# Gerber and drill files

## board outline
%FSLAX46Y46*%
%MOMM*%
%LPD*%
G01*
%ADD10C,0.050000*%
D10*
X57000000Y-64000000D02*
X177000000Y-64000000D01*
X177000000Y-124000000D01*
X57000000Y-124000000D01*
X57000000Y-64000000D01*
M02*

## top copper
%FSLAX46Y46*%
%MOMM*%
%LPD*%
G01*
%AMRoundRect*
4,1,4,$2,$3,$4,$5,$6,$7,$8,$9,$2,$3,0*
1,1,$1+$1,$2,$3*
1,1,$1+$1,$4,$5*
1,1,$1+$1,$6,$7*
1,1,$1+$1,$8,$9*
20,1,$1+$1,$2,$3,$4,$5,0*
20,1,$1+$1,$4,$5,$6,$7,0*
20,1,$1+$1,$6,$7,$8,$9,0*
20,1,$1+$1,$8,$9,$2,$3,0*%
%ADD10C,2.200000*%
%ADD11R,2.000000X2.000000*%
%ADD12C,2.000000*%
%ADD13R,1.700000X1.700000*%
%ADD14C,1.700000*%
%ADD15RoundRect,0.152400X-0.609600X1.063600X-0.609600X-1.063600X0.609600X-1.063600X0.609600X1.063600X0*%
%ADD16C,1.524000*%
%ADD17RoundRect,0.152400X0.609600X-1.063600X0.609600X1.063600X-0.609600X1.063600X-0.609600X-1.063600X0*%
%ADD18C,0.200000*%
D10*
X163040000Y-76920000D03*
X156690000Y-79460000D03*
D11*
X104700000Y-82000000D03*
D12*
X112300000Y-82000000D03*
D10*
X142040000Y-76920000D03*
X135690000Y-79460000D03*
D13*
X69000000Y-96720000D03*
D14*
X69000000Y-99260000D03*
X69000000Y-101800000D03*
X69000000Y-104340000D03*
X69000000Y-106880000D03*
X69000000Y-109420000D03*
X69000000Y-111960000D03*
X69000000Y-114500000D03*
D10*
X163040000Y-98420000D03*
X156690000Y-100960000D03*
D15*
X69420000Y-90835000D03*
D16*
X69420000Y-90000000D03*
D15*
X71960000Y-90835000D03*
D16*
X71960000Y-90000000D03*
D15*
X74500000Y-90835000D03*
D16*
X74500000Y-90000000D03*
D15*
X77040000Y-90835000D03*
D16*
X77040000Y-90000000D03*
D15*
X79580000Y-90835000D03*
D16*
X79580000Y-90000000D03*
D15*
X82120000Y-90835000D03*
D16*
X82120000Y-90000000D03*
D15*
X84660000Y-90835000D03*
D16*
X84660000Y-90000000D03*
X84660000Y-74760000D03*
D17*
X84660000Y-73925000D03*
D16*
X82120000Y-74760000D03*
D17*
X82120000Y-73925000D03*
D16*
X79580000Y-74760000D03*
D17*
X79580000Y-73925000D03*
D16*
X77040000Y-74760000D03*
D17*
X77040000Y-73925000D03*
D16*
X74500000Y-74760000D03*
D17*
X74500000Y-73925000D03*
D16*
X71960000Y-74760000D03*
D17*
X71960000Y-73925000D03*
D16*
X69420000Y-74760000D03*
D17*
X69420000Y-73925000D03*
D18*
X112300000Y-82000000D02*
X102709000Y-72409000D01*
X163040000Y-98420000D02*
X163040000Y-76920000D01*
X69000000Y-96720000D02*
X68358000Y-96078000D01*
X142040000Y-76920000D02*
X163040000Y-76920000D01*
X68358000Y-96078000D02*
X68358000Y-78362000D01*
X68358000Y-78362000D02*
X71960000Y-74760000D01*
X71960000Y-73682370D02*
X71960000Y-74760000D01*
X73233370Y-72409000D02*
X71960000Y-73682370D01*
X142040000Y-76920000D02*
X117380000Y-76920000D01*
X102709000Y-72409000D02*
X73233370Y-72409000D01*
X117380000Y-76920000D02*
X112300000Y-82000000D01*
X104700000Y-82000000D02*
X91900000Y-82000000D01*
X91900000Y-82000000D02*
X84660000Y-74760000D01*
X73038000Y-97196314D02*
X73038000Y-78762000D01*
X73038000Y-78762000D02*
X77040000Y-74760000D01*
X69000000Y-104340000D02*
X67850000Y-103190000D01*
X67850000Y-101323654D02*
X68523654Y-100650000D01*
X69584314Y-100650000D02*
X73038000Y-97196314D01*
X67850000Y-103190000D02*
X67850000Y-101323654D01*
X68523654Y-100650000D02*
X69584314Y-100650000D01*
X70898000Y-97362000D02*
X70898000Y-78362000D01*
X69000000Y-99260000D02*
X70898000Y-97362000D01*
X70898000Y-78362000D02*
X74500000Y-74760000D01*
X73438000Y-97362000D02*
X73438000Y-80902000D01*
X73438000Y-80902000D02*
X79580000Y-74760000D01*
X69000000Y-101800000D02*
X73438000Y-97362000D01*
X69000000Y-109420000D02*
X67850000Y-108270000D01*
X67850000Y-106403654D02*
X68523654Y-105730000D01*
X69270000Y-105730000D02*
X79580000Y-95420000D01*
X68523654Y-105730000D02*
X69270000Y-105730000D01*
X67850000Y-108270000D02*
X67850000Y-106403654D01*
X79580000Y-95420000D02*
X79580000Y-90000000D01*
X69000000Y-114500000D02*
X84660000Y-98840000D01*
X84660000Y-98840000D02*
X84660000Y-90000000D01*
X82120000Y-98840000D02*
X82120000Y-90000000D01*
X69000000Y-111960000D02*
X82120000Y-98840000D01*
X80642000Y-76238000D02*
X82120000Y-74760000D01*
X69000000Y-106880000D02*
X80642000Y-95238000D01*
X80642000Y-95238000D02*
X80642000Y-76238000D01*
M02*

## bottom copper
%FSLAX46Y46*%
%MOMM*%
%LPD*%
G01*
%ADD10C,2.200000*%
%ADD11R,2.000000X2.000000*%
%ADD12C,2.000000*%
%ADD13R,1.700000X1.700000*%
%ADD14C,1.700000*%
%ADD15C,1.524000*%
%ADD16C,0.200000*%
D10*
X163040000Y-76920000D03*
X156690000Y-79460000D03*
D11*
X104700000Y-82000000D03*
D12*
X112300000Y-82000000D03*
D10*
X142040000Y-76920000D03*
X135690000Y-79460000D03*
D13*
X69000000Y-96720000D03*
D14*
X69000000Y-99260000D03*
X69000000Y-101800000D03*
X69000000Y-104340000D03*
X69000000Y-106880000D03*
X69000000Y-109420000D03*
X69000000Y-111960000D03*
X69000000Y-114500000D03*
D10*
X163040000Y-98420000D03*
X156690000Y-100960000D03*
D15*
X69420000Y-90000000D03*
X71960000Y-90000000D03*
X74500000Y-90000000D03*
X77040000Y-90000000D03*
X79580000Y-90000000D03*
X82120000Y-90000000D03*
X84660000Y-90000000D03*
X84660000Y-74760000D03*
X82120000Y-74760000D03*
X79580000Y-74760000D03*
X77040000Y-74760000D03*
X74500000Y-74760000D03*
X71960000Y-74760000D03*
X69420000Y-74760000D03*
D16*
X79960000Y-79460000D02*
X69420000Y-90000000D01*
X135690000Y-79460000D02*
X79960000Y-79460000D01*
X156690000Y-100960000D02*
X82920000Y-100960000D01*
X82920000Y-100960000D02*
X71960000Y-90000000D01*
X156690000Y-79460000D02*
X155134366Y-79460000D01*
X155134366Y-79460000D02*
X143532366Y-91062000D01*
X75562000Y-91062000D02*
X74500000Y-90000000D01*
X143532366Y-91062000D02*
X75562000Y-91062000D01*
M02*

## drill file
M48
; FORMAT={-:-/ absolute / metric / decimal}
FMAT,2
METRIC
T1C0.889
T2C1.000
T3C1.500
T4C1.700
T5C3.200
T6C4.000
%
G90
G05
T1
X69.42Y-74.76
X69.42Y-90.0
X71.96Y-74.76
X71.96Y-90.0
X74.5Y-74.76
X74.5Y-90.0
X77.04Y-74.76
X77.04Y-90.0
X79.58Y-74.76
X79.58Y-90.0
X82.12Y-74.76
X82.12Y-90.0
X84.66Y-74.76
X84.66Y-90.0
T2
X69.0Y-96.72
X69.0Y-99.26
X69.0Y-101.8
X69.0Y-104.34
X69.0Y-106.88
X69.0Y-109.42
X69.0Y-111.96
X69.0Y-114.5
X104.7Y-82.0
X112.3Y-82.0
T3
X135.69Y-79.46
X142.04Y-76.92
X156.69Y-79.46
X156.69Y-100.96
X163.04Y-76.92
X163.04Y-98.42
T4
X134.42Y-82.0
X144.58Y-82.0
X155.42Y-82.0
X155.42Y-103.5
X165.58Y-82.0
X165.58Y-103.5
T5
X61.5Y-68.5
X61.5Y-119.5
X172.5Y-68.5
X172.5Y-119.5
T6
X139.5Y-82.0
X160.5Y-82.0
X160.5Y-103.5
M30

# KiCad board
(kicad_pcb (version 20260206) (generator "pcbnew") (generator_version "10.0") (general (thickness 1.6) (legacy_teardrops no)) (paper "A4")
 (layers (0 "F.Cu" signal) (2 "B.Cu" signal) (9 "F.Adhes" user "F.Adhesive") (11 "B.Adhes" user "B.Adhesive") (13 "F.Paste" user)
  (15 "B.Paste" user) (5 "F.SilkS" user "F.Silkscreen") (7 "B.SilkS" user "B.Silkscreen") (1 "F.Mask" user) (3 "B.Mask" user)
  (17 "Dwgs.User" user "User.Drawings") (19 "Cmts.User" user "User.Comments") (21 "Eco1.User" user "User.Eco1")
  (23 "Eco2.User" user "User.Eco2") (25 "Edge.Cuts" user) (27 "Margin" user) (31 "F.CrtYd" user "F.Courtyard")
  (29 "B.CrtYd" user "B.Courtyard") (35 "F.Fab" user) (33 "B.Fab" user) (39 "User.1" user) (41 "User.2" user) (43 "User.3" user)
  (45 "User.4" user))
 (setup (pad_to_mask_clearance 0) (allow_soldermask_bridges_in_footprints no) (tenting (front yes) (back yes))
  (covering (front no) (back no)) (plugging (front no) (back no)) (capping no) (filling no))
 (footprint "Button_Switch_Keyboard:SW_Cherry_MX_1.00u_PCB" (layer "F.Cu") (at 163.04 76.92)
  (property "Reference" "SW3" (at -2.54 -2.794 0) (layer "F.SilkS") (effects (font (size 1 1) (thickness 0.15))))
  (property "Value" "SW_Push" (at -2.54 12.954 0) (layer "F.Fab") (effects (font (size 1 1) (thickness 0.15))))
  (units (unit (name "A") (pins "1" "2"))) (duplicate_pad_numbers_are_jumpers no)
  (pad "" np_thru_hole circle (at -7.62 5.08) (size 1.7 1.7) (drill 1.7) (layers "*.Cu" "*.Mask"))
  (pad "" np_thru_hole circle (at -2.54 5.08) (size 4 4) (drill 4) (layers "*.Cu" "*.Mask"))
  (pad "" np_thru_hole circle (at 2.54 5.08) (size 1.7 1.7) (drill 1.7) (layers "*.Cu" "*.Mask"))
  (pad "1" thru_hole circle (at 0 0) (size 2.2 2.2) (drill 1.5) (layers "*.Cu" "*.Mask") (remove_unused_layers no) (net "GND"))
  (pad "2" thru_hole circle (at -6.35 2.54) (size 2.2 2.2) (drill 1.5) (layers "*.Cu" "*.Mask") (remove_unused_layers no)
   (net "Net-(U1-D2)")))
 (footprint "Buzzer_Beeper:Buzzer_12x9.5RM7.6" (layer "F.Cu") (at 104.7 82)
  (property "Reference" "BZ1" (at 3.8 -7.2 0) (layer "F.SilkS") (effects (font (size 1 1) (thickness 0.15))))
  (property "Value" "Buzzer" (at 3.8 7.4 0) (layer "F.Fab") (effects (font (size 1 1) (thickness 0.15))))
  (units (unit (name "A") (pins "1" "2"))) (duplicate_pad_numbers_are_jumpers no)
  (pad "1" thru_hole rect (at 0 0) (size 2 2) (drill 1) (layers "*.Cu" "*.Mask") (remove_unused_layers no) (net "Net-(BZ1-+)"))
  (pad "2" thru_hole circle (at 7.6 0) (size 2 2) (drill 1) (layers "*.Cu" "*.Mask") (remove_unused_layers no) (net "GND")))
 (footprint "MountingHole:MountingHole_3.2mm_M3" (layer "F.Cu") (at 172.5 119.5)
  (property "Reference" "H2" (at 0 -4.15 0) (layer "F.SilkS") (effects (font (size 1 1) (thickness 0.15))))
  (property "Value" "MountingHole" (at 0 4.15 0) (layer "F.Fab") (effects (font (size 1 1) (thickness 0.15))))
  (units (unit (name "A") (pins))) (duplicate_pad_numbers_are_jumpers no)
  (pad "" np_thru_hole circle (at 0 0) (size 3.2 3.2) (drill 3.2) (layers "*.Cu" "*.Mask")))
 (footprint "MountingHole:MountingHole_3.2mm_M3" (layer "F.Cu") (at 172.5 68.5)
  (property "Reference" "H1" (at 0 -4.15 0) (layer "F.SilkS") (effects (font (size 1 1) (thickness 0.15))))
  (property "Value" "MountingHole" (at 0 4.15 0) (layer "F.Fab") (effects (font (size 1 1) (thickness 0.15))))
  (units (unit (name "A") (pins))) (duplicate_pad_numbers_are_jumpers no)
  (pad "" np_thru_hole circle (at 0 0) (size 3.2 3.2) (drill 3.2) (layers "*.Cu" "*.Mask")))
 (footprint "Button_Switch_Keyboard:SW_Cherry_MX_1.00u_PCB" (layer "F.Cu") (at 142.04 76.92)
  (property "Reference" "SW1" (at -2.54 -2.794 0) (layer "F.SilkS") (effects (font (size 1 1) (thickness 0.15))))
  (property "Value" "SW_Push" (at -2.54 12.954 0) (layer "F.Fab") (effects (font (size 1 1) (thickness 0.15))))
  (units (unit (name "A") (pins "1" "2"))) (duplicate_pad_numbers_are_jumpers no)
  (pad "" np_thru_hole circle (at -7.62 5.08) (size 1.7 1.7) (drill 1.7) (layers "*.Cu" "*.Mask"))
  (pad "" np_thru_hole circle (at -2.54 5.08) (size 4 4) (drill 4) (layers "*.Cu" "*.Mask"))
  (pad "" np_thru_hole circle (at 2.54 5.08) (size 1.7 1.7) (drill 1.7) (layers "*.Cu" "*.Mask"))
  (pad "1" thru_hole circle (at 0 0) (size 2.2 2.2) (drill 1.5) (layers "*.Cu" "*.Mask") (remove_unused_layers no) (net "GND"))
  (pad "2" thru_hole circle (at -6.35 2.54) (size 2.2 2.2) (drill 1.5) (layers "*.Cu" "*.Mask") (remove_unused_layers no)
   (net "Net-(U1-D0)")))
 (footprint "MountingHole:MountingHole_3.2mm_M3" (layer "F.Cu") (at 61.5 68.5)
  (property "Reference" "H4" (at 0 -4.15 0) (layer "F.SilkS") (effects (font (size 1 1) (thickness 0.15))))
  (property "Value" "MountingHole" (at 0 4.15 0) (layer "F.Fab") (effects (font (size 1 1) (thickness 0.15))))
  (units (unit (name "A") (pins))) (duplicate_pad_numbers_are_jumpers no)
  (pad "" np_thru_hole circle (at 0 0) (size 3.2 3.2) (drill 3.2) (layers "*.Cu" "*.Mask")))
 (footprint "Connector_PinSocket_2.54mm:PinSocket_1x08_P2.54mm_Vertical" (layer "F.Cu") (at 69 96.72)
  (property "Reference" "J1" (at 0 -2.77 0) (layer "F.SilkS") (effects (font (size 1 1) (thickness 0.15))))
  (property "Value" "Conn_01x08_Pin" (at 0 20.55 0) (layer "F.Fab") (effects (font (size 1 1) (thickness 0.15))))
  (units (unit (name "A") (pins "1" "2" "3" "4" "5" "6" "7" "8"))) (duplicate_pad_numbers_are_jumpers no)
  (pad "1" thru_hole rect (at 0 0) (size 1.7 1.7) (drill 1) (layers "*.Cu" "*.Mask") (remove_unused_layers no) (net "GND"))
  (pad "2" thru_hole circle (at 0 2.54) (size 1.7 1.7) (drill 1) (layers "*.Cu" "*.Mask") (remove_unused_layers no) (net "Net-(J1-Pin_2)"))
  (pad "3" thru_hole circle (at 0 5.08) (size 1.7 1.7) (drill 1) (layers "*.Cu" "*.Mask") (remove_unused_layers no) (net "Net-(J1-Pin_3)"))
  (pad "4" thru_hole circle (at 0 7.62) (size 1.7 1.7) (drill 1) (layers "*.Cu" "*.Mask") (remove_unused_layers no) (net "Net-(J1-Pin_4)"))
  (pad "5" thru_hole circle (at 0 10.16) (size 1.7 1.7) (drill 1) (layers "*.Cu" "*.Mask") (remove_unused_layers no) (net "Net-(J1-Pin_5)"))
  (pad "6" thru_hole circle (at 0 12.7) (size 1.7 1.7) (drill 1) (layers "*.Cu" "*.Mask") (remove_unused_layers no) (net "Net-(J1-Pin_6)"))
  (pad "7" thru_hole circle (at 0 15.24) (size 1.7 1.7) (drill 1) (layers "*.Cu" "*.Mask") (remove_unused_layers no) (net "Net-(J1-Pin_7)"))
  (pad "8" thru_hole circle (at 0 17.78) (size 1.7 1.7) (drill 1) (layers "*.Cu" "*.Mask") (remove_unused_layers no) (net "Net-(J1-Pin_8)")))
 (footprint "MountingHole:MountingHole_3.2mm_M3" (layer "F.Cu") (at 61.5 119.5)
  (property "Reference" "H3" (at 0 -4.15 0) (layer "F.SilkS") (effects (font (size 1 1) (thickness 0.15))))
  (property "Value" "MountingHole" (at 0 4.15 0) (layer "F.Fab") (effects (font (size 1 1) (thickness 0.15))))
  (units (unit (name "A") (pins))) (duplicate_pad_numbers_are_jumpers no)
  (pad "" np_thru_hole circle (at 0 0) (size 3.2 3.2) (drill 3.2) (layers "*.Cu" "*.Mask")))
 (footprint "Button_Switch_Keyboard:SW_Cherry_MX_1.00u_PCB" (layer "F.Cu") (at 163.04 98.42)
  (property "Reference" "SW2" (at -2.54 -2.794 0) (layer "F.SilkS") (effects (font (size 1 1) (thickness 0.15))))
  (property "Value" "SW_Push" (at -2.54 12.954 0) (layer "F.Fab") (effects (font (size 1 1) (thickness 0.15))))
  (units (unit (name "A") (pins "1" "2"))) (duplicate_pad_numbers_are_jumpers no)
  (pad "" np_thru_hole circle (at -7.62 5.08) (size 1.7 1.7) (drill 1.7) (layers "*.Cu" "*.Mask"))
  (pad "" np_thru_hole circle (at -2.54 5.08) (size 4 4) (drill 4) (layers "*.Cu" "*.Mask"))
  (pad "" np_thru_hole circle (at 2.54 5.08) (size 1.7 1.7) (drill 1.7) (layers "*.Cu" "*.Mask"))
  (pad "1" thru_hole circle (at 0 0) (size 2.2 2.2) (drill 1.5) (layers "*.Cu" "*.Mask") (remove_unused_layers no) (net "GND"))
  (pad "2" thru_hole circle (at -6.35 2.54) (size 2.2 2.2) (drill 1.5) (layers "*.Cu" "*.Mask") (remove_unused_layers no)
   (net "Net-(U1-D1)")))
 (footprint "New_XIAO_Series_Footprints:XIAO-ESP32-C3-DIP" (layer "F.Cu") (at 77.04 82.38 180)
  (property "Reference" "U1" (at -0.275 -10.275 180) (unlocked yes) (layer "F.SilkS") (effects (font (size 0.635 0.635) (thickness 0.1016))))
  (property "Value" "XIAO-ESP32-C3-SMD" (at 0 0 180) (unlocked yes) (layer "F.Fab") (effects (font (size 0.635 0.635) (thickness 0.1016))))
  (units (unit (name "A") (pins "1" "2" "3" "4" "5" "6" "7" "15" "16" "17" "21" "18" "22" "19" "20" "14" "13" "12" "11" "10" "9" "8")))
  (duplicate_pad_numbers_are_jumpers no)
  (pad "1" smd roundrect (at 7.62 -8.455 270) (size 2.432 1.524) (layers "F.Cu" "F.Mask") (roundrect_rratio 0.1) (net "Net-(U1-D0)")
   (thermal_bridge_angle 45))
  (pad "1" thru_hole circle (at 7.62 -7.62 270) (size 1.524 1.524) (drill 0.889) (layers "*.Cu" "*.Mask") (remove_unused_layers no)
   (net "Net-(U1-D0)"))
  (pad "2" smd roundrect (at 5.08 -8.455 270) (size 2.432 1.524) (layers "F.Cu" "F.Mask") (roundrect_rratio 0.1) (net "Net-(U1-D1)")
   (thermal_bridge_angle 45))
  (pad "2" thru_hole circle (at 5.08 -7.62 270) (size 1.524 1.524) (drill 0.889) (layers "*.Cu" "*.Mask") (remove_unused_layers no)
   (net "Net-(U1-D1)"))
  (pad "3" smd roundrect (at 2.54 -8.455 270) (size 2.432 1.524) (layers "F.Cu" "F.Mask") (roundrect_rratio 0.1) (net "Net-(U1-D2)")
   (thermal_bridge_angle 45))
  (pad "3" thru_hole circle (at 2.54 -7.62 270) (size 1.524 1.524) (drill 0.889) (layers "*.Cu" "*.Mask") (remove_unused_layers no)
   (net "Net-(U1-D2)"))
  (pad "4" smd roundrect (at 0 -8.455 270) (size 2.432 1.524) (layers "F.Cu" "F.Mask") (roundrect_rratio 0.1)
   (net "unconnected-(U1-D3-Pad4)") (thermal_bridge_angle 45))
  (pad "4" thru_hole circle (at 0 -7.62 270) (size 1.524 1.524) (drill 0.889) (layers "*.Cu" "*.Mask") (remove_unused_layers no)
   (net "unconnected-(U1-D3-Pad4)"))
  (pad "5" smd roundrect (at -2.54 -8.455 270) (size 2.432 1.524) (layers "F.Cu" "F.Mask") (roundrect_rratio 0.1) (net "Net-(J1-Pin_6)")
   (thermal_bridge_angle 45))
  (pad "5" thru_hole circle (at -2.54 -7.62 270) (size 1.524 1.524) (drill 0.889) (layers "*.Cu" "*.Mask") (remove_unused_layers no)
   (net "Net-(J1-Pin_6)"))
  (pad "6" smd roundrect (at -5.08 -8.455 270) (size 2.432 1.524) (layers "F.Cu" "F.Mask") (roundrect_rratio 0.1) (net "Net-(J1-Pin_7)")
   (thermal_bridge_angle 45))
  (pad "6" thru_hole circle (at -5.08 -7.62 270) (size 1.524 1.524) (drill 0.889) (layers "*.Cu" "*.Mask") (remove_unused_layers no)
   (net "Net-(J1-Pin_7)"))
  (pad "7" smd roundrect (at -7.62 -8.455 270) (size 2.432 1.524) (layers "F.Cu" "F.Mask") (roundrect_rratio 0.1) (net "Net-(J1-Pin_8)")
   (thermal_bridge_angle 45))
  (pad "7" thru_hole circle (at -7.62 -7.62 270) (size 1.524 1.524) (drill 0.889) (layers "*.Cu" "*.Mask") (remove_unused_layers no)
   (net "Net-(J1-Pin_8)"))
  (pad "8" thru_hole circle (at -7.62 7.62 90) (size 1.524 1.524) (drill 0.889) (layers "*.Cu" "*.Mask") (remove_unused_layers no)
   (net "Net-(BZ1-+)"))
  (pad "8" smd roundrect (at -7.62 8.455 90) (size 2.432 1.524) (layers "F.Cu" "F.Mask") (roundrect_rratio 0.1) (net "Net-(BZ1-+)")
   (thermal_bridge_angle 45))
  (pad "9" thru_hole circle (at -5.08 7.62 90) (size 1.524 1.524) (drill 0.889) (layers "*.Cu" "*.Mask") (remove_unused_layers no)
   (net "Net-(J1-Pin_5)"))
  (pad "9" smd roundrect (at -5.08 8.455 90) (size 2.432 1.524) (layers "F.Cu" "F.Mask") (roundrect_rratio 0.1) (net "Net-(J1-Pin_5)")
   (thermal_bridge_angle 45))
  (pad "10" thru_hole circle (at -2.54 7.62 90) (size 1.524 1.524) (drill 0.889) (layers "*.Cu" "*.Mask") (remove_unused_layers no)
   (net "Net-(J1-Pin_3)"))
  (pad "10" smd roundrect (at -2.54 8.455 90) (size 2.432 1.524) (layers "F.Cu" "F.Mask") (roundrect_rratio 0.1) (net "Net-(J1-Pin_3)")
   (thermal_bridge_angle 45))
  (pad "11" thru_hole circle (at 0 7.62 90) (size 1.524 1.524) (drill 0.889) (layers "*.Cu" "*.Mask") (remove_unused_layers no)
   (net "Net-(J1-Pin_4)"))
  (pad "11" smd roundrect (at 0 8.455 90) (size 2.432 1.524) (layers "F.Cu" "F.Mask") (roundrect_rratio 0.1) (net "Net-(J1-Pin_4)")
   (thermal_bridge_angle 45))
  (pad "12" thru_hole circle (at 2.54 7.62 90) (size 1.524 1.524) (drill 0.889) (layers "*.Cu" "*.Mask") (remove_unused_layers no)
   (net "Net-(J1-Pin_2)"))
  (pad "12" smd roundrect (at 2.54 8.455 90) (size 2.432 1.524) (layers "F.Cu" "F.Mask") (roundrect_rratio 0.1) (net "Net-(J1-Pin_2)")
   (thermal_bridge_angle 45))
  (pad "13" thru_hole circle (at 5.08 7.62 90) (size 1.524 1.524) (drill 0.889) (layers "*.Cu" "*.Mask") (remove_unused_layers no)
   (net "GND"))
  (pad "13" smd roundrect (at 5.08 8.455 90) (size 2.432 1.524) (layers "F.Cu" "F.Mask") (roundrect_rratio 0.1) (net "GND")
   (thermal_bridge_angle 45))
  (pad "14" thru_hole circle (at 7.62 7.62 90) (size 1.524 1.524) (drill 0.889) (layers "*.Cu" "*.Mask") (remove_unused_layers no)
   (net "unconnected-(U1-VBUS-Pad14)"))
  (pad "14" smd roundrect (at 7.62 8.455 90) (size 2.432 1.524) (layers "F.Cu" "F.Mask") (roundrect_rratio 0.1)
   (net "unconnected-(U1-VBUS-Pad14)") (thermal_bridge_angle 45)))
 (gr_rect (start 57 64) (end 177 124) (stroke (width 0.05) (type default)) (fill no) (layer "Edge.Cuts"))
 (segment (start 112.3 82) (end 102.709 72.409) (width 0.2) (layer "F.Cu") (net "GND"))
 (segment (start 163.04 98.42) (end 163.04 76.92) (width 0.2) (layer "F.Cu") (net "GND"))
 (segment (start 69 96.72) (end 68.358 96.078) (width 0.2) (layer "F.Cu") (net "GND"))
 (segment (start 142.04 76.92) (end 163.04 76.92) (width 0.2) (layer "F.Cu") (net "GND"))
 (segment (start 68.358 96.078) (end 68.358 78.362) (width 0.2) (layer "F.Cu") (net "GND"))
 (segment (start 68.358 78.362) (end 71.96 74.76) (width 0.2) (layer "F.Cu") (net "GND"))
 (segment (start 71.96 73.68237) (end 71.96 74.76) (width 0.2) (layer "F.Cu") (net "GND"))
 (segment (start 73.23337 72.409) (end 71.96 73.68237) (width 0.2) (layer "F.Cu") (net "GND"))
 (segment (start 142.04 76.92) (end 117.38 76.92) (width 0.2) (layer "F.Cu") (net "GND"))
 (segment (start 102.709 72.409) (end 73.23337 72.409) (width 0.2) (layer "F.Cu") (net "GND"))
 (segment (start 117.38 76.92) (end 112.3 82) (width 0.2) (layer "F.Cu") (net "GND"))
 (segment (start 104.7 82) (end 91.9 82) (width 0.2) (layer "F.Cu") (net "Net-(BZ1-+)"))
 (segment (start 91.9 82) (end 84.66 74.76) (width 0.2) (layer "F.Cu") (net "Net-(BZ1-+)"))
 (segment (start 73.038 97.196314) (end 73.038 78.762) (width 0.2) (layer "F.Cu") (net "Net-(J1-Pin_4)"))
 (segment (start 73.038 78.762) (end 77.04 74.76) (width 0.2) (layer "F.Cu") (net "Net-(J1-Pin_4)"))
 (segment (start 69 104.34) (end 67.85 103.19) (width 0.2) (layer "F.Cu") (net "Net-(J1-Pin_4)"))
 (segment (start 67.85 101.323654) (end 68.523654 100.65) (width 0.2) (layer "F.Cu") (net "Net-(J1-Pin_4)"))
 (segment (start 69.584314 100.65) (end 73.038 97.196314) (width 0.2) (layer "F.Cu") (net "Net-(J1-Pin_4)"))
 (segment (start 67.85 103.19) (end 67.85 101.323654) (width 0.2) (layer "F.Cu") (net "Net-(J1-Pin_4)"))
 (segment (start 68.523654 100.65) (end 69.584314 100.65) (width 0.2) (layer "F.Cu") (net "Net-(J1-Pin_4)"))
 (segment (start 70.898 97.362) (end 70.898 78.362) (width 0.2) (layer "F.Cu") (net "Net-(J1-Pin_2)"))
 (segment (start 69 99.26) (end 70.898 97.362) (width 0.2) (layer "F.Cu") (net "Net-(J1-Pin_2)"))
 (segment (start 70.898 78.362) (end 74.5 74.76) (width 0.2) (layer "F.Cu") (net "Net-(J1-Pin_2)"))
 (segment (start 73.438 97.362) (end 73.438 80.902) (width 0.2) (layer "F.Cu") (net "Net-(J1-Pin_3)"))
 (segment (start 73.438 80.902) (end 79.58 74.76) (width 0.2) (layer "F.Cu") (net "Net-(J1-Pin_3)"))
 (segment (start 69 101.8) (end 73.438 97.362) (width 0.2) (layer "F.Cu") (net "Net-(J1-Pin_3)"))
 (segment (start 69 109.42) (end 67.85 108.27) (width 0.2) (layer "F.Cu") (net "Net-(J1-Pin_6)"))
 (segment (start 67.85 106.403654) (end 68.523654 105.73) (width 0.2) (layer "F.Cu") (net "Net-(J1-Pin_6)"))
 (segment (start 69.27 105.73) (end 79.58 95.42) (width 0.2) (layer "F.Cu") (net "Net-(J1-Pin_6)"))
 (segment (start 68.523654 105.73) (end 69.27 105.73) (width 0.2) (layer "F.Cu") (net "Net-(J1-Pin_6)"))
 (segment (start 67.85 108.27) (end 67.85 106.403654) (width 0.2) (layer "F.Cu") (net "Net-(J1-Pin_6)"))
 (segment (start 79.58 95.42) (end 79.58 90) (width 0.2) (layer "F.Cu") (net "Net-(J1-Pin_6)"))
 (segment (start 69 114.5) (end 84.66 98.84) (width 0.2) (layer "F.Cu") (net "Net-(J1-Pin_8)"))
 (segment (start 84.66 98.84) (end 84.66 90) (width 0.2) (layer "F.Cu") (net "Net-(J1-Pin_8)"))
 (segment (start 82.12 98.84) (end 82.12 90) (width 0.2) (layer "F.Cu") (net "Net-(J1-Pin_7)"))
 (segment (start 69 111.96) (end 82.12 98.84) (width 0.2) (layer "F.Cu") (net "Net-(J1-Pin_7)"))
 (segment (start 80.642 76.238) (end 82.12 74.76) (width 0.2) (layer "F.Cu") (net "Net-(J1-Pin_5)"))
 (segment (start 69 106.88) (end 80.642 95.238) (width 0.2) (layer "F.Cu") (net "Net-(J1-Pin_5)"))
 (segment (start 80.642 95.238) (end 80.642 76.238) (width 0.2) (layer "F.Cu") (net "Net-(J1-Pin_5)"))
 (segment (start 79.96 79.46) (end 69.42 90) (width 0.2) (layer "B.Cu") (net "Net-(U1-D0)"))
 (segment (start 135.69 79.46) (end 79.96 79.46) (width 0.2) (layer "B.Cu") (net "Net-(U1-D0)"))
 (segment (start 156.69 100.96) (end 82.92 100.96) (width 0.2) (layer "B.Cu") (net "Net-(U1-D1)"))
 (segment (start 82.92 100.96) (end 71.96 90) (width 0.2) (layer "B.Cu") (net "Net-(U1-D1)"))
 (segment (start 156.69 79.46) (end 155.134366 79.46) (width 0.2) (layer "B.Cu") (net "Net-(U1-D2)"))
 (segment (start 155.134366 79.46) (end 143.532366 91.062) (width 0.2) (layer "B.Cu") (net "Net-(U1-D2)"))
 (segment (start 75.562 91.062) (end 74.5 90) (width 0.2) (layer "B.Cu") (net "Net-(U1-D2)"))
 (segment (start 143.532366 91.062) (end 75.562 91.062) (width 0.2) (layer "B.Cu") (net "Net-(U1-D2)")))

